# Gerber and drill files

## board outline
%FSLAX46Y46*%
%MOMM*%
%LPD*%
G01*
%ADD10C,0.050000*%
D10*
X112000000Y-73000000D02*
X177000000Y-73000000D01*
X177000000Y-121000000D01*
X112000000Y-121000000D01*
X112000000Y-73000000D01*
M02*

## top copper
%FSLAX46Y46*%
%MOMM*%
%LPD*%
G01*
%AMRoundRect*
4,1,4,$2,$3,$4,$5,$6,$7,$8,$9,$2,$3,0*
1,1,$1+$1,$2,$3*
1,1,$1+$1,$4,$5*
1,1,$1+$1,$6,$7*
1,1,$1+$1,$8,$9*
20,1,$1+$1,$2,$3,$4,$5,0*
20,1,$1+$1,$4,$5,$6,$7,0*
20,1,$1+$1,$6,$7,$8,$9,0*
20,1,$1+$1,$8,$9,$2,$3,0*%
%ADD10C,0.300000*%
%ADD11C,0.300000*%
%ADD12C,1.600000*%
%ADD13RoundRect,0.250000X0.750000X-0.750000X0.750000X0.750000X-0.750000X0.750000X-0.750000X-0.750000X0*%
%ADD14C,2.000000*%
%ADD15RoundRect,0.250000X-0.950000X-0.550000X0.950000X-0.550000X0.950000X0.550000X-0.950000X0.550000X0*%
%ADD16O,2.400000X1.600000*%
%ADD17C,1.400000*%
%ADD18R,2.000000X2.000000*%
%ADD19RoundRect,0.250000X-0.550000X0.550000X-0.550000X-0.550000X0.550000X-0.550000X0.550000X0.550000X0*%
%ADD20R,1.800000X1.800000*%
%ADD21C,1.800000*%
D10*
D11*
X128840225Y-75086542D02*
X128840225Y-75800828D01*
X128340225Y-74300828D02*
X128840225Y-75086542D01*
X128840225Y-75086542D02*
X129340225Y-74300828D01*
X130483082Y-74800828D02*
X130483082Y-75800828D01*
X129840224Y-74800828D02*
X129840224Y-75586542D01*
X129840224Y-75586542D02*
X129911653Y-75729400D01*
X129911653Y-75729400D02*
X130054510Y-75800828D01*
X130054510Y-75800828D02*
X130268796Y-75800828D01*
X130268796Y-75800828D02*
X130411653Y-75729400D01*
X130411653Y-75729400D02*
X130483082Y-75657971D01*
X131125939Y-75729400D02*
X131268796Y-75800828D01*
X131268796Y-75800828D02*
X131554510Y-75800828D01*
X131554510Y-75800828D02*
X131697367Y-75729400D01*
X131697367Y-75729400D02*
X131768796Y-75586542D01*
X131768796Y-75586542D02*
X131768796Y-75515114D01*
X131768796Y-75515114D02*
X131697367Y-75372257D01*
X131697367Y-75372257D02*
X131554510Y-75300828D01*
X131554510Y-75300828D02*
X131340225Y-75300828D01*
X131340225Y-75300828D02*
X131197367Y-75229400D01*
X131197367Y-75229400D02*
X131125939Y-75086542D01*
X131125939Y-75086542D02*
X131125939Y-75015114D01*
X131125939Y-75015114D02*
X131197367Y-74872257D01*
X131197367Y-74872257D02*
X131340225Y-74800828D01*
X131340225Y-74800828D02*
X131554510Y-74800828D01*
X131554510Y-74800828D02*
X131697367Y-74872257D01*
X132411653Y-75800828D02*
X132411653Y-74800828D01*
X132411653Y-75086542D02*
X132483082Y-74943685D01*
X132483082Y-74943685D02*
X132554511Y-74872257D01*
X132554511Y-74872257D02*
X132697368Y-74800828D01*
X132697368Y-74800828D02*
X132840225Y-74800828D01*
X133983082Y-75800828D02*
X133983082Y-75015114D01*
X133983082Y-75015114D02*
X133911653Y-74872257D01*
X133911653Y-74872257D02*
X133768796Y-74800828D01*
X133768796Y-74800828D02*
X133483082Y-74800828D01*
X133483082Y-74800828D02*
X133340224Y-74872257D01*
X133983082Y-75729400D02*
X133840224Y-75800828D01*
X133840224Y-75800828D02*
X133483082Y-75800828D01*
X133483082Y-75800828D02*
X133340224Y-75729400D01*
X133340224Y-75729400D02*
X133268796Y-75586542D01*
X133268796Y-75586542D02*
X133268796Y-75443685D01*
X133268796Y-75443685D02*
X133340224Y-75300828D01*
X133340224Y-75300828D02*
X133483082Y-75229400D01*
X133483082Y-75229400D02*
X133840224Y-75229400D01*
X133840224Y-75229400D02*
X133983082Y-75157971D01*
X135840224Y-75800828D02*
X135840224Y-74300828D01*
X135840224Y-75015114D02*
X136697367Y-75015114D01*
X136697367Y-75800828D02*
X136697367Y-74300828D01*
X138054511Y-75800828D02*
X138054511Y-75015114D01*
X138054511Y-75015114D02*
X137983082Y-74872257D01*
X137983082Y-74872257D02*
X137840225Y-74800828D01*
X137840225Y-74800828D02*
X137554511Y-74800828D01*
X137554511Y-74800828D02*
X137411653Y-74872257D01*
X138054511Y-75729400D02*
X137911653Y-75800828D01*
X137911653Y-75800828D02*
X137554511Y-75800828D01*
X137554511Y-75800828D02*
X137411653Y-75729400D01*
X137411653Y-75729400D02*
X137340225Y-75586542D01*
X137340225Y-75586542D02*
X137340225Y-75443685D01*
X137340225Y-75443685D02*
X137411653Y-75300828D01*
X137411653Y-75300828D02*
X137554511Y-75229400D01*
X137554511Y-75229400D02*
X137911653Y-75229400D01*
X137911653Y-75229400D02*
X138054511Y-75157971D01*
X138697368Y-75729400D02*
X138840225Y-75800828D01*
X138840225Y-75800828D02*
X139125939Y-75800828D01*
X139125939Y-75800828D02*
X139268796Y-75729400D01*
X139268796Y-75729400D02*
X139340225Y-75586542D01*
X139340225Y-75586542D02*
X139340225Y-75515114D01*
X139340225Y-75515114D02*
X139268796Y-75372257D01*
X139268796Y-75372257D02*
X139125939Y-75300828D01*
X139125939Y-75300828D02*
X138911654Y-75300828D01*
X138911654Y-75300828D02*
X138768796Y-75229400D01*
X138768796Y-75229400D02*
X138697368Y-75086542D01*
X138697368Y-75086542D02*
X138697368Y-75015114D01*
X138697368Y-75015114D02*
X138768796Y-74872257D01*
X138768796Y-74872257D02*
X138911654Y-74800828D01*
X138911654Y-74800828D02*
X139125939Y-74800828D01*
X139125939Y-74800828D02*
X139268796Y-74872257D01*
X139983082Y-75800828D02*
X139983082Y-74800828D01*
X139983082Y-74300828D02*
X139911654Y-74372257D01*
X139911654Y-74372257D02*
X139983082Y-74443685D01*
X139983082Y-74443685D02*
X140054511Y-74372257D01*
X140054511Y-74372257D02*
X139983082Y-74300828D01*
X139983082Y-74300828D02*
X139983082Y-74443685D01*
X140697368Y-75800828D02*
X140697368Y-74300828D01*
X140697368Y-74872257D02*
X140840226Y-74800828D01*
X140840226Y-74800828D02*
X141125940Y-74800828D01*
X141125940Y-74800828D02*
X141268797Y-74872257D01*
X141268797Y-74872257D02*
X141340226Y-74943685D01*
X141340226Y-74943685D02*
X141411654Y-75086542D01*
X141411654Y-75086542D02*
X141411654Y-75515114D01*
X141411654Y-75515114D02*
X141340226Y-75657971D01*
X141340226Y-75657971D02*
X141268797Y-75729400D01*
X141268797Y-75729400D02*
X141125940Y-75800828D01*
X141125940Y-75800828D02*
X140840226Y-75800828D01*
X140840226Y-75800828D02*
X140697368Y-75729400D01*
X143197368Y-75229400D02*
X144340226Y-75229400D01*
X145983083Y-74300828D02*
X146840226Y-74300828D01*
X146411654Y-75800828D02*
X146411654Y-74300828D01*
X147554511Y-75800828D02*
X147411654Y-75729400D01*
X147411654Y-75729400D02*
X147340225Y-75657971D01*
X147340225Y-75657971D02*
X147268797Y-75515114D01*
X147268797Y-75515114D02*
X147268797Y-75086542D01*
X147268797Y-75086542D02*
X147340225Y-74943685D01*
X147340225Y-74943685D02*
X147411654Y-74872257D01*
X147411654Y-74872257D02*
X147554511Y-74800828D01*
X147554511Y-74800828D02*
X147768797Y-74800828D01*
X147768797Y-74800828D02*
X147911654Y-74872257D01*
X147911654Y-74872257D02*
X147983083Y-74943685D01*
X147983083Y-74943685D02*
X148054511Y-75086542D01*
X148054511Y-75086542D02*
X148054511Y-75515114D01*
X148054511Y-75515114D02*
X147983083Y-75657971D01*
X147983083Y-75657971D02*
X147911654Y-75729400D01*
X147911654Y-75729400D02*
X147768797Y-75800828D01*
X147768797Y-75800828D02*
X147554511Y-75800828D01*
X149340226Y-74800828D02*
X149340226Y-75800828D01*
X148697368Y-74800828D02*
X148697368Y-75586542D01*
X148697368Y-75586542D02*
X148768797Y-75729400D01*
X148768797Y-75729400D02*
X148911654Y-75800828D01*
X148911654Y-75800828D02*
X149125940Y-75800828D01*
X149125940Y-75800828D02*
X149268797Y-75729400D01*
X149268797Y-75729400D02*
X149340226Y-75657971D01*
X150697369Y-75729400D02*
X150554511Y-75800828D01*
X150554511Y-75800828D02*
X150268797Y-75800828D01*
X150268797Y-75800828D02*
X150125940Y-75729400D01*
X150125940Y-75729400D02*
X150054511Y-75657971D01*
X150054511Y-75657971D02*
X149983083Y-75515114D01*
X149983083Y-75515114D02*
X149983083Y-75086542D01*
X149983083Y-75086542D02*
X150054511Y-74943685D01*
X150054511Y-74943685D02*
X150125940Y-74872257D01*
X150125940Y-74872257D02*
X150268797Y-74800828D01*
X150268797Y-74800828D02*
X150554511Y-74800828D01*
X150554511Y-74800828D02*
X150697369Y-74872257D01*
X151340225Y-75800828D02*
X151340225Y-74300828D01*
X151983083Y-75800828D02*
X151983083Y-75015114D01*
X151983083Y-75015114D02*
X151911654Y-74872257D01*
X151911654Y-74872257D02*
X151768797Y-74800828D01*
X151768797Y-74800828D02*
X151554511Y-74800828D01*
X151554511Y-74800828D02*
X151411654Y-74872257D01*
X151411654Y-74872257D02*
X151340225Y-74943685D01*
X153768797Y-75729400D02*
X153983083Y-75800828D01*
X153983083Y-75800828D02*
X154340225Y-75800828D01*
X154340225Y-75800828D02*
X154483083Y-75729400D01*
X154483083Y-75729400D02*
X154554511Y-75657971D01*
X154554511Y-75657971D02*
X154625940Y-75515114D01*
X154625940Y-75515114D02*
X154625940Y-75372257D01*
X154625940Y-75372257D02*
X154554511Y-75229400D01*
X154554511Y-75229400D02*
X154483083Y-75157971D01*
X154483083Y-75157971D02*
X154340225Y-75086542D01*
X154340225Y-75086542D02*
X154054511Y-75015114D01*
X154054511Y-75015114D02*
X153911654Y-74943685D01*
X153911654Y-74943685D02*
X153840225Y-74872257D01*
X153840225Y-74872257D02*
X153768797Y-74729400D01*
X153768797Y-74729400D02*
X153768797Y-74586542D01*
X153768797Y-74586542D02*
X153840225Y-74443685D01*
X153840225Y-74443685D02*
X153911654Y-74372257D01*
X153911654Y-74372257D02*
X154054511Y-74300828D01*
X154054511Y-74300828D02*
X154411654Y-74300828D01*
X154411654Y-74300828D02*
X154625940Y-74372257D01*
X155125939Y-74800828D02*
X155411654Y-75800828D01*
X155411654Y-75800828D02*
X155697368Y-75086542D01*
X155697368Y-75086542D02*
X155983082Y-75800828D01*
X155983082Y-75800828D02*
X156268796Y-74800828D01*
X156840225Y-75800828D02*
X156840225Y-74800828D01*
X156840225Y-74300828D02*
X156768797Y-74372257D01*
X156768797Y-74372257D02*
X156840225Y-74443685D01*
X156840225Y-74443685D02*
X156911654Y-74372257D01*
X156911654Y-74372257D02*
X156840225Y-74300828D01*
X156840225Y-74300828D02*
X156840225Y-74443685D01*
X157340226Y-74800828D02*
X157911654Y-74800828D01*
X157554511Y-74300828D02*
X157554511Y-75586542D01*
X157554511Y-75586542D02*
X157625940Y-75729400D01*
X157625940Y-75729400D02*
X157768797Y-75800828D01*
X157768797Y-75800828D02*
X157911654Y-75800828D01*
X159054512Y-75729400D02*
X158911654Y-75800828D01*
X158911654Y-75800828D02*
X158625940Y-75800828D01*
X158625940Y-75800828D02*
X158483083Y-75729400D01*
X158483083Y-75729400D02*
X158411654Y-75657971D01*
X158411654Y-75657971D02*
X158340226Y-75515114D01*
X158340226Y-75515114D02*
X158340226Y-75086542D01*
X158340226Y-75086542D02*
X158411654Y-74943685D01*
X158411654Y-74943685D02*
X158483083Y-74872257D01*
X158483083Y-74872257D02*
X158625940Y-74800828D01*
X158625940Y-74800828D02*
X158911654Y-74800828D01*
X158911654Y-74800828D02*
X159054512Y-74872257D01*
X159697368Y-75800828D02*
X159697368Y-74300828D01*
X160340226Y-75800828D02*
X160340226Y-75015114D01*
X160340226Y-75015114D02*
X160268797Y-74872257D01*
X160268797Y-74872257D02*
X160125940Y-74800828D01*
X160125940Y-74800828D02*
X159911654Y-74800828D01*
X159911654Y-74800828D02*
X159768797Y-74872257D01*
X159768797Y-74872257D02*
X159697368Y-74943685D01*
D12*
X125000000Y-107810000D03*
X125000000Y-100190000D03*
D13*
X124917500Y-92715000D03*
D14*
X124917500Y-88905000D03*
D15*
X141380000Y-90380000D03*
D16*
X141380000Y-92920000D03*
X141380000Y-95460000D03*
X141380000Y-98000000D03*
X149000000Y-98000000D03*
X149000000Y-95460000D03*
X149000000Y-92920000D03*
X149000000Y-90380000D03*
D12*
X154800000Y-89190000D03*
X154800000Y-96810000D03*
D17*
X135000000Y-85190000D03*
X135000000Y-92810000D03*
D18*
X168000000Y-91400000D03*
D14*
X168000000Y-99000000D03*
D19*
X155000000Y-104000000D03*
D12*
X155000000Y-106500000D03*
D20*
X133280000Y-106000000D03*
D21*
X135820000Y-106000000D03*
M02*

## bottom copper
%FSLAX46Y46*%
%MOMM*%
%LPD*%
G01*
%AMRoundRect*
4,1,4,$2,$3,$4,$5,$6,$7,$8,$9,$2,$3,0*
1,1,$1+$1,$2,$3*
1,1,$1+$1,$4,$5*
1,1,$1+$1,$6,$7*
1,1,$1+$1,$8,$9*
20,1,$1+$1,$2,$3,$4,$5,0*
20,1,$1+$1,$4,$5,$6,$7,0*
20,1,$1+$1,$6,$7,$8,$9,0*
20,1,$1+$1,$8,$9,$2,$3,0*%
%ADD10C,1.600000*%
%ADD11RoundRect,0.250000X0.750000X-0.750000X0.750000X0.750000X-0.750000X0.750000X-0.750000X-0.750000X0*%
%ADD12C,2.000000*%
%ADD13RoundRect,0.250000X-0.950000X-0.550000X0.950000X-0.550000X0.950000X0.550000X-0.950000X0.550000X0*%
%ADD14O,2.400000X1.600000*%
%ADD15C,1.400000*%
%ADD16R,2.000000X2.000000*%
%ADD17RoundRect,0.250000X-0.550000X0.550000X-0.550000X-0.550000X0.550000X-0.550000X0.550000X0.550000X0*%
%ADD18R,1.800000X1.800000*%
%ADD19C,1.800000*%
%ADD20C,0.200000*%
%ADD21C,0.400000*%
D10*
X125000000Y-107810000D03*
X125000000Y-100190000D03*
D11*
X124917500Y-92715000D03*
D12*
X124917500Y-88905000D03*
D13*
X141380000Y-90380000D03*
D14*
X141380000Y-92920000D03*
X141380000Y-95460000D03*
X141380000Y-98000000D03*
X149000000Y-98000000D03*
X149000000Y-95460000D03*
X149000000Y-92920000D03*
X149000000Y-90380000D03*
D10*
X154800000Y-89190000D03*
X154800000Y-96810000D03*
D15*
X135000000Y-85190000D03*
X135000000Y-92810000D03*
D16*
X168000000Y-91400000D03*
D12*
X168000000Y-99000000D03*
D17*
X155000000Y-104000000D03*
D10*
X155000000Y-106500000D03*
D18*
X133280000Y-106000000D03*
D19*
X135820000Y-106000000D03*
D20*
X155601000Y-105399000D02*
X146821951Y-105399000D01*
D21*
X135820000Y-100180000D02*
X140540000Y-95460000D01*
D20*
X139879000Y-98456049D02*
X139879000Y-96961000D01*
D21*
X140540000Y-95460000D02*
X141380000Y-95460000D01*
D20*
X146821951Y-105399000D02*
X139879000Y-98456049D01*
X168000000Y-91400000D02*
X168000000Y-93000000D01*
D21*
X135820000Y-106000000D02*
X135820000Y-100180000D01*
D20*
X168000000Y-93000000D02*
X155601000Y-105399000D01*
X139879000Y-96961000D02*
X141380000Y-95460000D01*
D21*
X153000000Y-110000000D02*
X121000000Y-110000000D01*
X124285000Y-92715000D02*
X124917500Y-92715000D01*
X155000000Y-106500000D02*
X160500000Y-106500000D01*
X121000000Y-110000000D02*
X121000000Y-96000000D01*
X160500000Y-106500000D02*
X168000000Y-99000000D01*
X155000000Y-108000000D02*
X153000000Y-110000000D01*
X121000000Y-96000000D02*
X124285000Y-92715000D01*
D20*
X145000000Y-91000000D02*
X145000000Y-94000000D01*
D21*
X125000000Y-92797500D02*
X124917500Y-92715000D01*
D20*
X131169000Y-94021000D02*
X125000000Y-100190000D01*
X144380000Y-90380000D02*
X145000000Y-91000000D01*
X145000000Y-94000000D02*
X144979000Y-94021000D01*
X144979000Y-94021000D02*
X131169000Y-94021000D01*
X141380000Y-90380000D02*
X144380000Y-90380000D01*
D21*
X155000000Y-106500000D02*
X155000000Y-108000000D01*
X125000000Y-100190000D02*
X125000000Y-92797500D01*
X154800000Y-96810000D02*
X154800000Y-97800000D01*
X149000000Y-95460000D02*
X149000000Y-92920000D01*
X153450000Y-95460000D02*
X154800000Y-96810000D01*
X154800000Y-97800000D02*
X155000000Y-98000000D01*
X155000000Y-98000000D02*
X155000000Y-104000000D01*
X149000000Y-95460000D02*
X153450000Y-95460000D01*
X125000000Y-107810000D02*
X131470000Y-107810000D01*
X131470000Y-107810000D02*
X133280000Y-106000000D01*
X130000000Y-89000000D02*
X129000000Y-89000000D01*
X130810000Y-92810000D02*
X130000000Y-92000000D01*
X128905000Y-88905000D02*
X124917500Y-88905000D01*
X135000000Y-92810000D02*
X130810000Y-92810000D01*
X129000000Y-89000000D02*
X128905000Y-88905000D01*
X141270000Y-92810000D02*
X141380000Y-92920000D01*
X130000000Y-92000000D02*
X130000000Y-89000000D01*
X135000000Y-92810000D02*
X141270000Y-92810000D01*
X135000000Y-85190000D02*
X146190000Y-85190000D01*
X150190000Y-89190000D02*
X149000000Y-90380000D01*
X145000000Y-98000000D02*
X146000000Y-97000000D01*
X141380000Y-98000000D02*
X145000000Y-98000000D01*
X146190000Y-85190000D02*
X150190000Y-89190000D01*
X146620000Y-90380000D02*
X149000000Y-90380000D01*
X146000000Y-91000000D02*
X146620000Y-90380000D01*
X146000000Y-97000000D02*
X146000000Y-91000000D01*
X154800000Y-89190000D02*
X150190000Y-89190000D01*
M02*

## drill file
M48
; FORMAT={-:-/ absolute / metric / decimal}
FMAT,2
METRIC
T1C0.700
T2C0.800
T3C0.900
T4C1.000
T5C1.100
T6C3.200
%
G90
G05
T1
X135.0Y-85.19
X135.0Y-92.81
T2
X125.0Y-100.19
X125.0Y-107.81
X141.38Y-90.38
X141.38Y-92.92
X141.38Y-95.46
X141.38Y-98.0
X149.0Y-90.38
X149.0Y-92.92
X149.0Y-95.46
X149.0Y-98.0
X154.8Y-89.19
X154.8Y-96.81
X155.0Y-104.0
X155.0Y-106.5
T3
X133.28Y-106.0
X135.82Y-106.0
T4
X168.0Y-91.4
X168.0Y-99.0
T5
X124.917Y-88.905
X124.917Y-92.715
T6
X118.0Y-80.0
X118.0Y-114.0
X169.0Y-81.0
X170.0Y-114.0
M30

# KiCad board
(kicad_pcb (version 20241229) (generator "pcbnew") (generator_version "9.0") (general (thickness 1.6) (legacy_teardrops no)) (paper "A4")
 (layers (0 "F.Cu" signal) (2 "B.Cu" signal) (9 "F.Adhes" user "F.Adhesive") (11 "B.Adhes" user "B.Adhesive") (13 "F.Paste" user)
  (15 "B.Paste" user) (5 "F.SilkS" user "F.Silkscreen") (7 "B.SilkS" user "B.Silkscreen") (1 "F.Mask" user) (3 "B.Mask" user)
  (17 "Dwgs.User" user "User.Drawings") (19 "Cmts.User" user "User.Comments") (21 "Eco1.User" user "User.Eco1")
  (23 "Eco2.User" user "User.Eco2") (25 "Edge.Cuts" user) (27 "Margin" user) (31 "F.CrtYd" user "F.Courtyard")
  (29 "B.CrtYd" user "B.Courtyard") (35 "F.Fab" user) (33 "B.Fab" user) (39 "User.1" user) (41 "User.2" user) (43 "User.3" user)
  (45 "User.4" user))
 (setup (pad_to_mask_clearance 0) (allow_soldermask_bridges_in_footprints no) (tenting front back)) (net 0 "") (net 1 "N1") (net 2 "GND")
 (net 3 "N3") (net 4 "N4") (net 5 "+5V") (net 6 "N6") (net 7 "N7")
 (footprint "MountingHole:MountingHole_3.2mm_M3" (layer "F.Cu") (at 169 81)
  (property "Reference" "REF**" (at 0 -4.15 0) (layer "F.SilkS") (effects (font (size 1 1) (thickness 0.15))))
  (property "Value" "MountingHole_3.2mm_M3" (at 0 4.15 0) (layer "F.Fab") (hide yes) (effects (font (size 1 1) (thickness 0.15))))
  (pad "" np_thru_hole circle (at 0 0) (size 3.2 3.2) (drill 3.2) (layers "*.Cu" "*.Mask")))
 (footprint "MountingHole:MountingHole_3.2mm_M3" (layer "F.Cu") (at 118 114)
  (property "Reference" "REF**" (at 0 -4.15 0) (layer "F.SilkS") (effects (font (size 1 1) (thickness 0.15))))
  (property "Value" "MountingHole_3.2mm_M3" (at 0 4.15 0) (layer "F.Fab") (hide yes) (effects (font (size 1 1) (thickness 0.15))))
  (pad "" np_thru_hole circle (at 0 0) (size 3.2 3.2) (drill 3.2) (layers "*.Cu" "*.Mask")))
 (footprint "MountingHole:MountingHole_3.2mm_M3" (layer "F.Cu") (at 118 80)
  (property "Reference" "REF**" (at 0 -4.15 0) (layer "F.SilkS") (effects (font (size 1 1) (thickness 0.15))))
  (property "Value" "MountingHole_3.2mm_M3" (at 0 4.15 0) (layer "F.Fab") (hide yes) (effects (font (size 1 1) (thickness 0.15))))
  (pad "" np_thru_hole circle (at 0 0) (size 3.2 3.2) (drill 3.2) (layers "*.Cu" "*.Mask")))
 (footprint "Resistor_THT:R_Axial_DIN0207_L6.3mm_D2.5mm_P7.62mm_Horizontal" (layer "F.Cu") (at 125 107.81 90)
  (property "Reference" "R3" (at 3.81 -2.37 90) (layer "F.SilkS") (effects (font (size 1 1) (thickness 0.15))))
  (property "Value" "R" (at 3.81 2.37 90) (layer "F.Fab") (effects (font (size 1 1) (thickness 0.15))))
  (pad "1" thru_hole circle (at 0 0 90) (size 1.6 1.6) (drill 0.8) (layers "*.Cu" "*.Mask") (remove_unused_layers no) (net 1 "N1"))
  (pad "2" thru_hole circle (at 7.62 0 90) (size 1.6 1.6) (drill 0.8) (layers "*.Cu" "*.Mask") (remove_unused_layers no) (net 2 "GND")))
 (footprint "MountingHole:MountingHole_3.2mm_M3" (layer "F.Cu") (at 170 114)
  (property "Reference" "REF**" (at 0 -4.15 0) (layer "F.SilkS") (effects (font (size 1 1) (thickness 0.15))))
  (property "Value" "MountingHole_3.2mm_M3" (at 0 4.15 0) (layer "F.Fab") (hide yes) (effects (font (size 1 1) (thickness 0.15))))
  (pad "" np_thru_hole circle (at 0 0) (size 3.2 3.2) (drill 3.2) (layers "*.Cu" "*.Mask")))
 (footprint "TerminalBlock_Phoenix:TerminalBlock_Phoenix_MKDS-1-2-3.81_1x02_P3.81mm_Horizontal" (layer "F.Cu") (at 124.9175 92.715 90)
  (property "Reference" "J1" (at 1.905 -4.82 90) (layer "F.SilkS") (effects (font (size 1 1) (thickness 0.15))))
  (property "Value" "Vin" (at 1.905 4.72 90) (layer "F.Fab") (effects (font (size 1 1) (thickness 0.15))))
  (pad "1" thru_hole roundrect (at 0 0 90) (size 2 2) (drill 1.1) (layers "*.Cu" "*.Mask") (remove_unused_layers no)
   (roundrect_rratio 0.125) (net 2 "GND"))
  (pad "2" thru_hole circle (at 3.81 0 90) (size 2 2) (drill 1.1) (layers "*.Cu" "*.Mask") (remove_unused_layers no) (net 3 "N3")))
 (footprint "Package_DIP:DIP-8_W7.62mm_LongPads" (layer "F.Cu") (at 141.38 90.38)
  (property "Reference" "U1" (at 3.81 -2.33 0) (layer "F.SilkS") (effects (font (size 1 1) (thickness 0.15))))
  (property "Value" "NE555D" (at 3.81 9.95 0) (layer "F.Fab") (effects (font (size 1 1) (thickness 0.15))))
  (pad "1" thru_hole roundrect (at 0 0) (size 2.4 1.6) (drill 0.8) (layers "*.Cu" "*.Mask") (remove_unused_layers no)
   (roundrect_rratio 0.15625) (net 2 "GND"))
  (pad "2" thru_hole oval (at 0 2.54) (size 2.4 1.6) (drill 0.8) (layers "*.Cu" "*.Mask") (remove_unused_layers no) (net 3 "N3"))
  (pad "3" thru_hole oval (at 0 5.08) (size 2.4 1.6) (drill 0.8) (layers "*.Cu" "*.Mask") (remove_unused_layers no) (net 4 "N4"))
  (pad "4" thru_hole oval (at 0 7.62) (size 2.4 1.6) (drill 0.8) (layers "*.Cu" "*.Mask") (remove_unused_layers no) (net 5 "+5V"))
  (pad "5" thru_hole oval (at 7.62 7.62) (size 2.4 1.6) (drill 0.8) (layers "*.Cu" "*.Mask") (remove_unused_layers no) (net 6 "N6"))
  (pad "6" thru_hole oval (at 7.62 5.08) (size 2.4 1.6) (drill 0.8) (layers "*.Cu" "*.Mask") (remove_unused_layers no) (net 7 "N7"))
  (pad "7" thru_hole oval (at 7.62 2.54) (size 2.4 1.6) (drill 0.8) (layers "*.Cu" "*.Mask") (remove_unused_layers no) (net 7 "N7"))
  (pad "8" thru_hole oval (at 7.62 0) (size 2.4 1.6) (drill 0.8) (layers "*.Cu" "*.Mask") (remove_unused_layers no) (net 5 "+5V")))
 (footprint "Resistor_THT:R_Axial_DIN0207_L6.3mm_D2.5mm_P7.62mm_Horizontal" (layer "F.Cu") (at 154.8 89.19 -90)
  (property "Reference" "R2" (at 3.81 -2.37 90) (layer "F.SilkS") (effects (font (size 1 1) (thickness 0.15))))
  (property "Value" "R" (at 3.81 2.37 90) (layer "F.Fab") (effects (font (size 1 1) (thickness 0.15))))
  (pad "1" thru_hole circle (at 0 0 270) (size 1.6 1.6) (drill 0.8) (layers "*.Cu" "*.Mask") (remove_unused_layers no) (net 5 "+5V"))
  (pad "2" thru_hole circle (at 7.62 0 270) (size 1.6 1.6) (drill 0.8) (layers "*.Cu" "*.Mask") (remove_unused_layers no) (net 7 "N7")))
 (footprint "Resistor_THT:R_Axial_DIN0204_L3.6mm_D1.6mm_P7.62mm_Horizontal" (layer "F.Cu") (at 135 85.19 -90)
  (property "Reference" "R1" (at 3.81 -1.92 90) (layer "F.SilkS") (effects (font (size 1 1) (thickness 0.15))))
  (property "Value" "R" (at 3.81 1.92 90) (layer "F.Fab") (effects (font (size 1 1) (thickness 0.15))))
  (pad "1" thru_hole circle (at 0 0 270) (size 1.4 1.4) (drill 0.7) (layers "*.Cu" "*.Mask") (remove_unused_layers no) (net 5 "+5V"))
  (pad "2" thru_hole circle (at 7.62 0 270) (size 1.4 1.4) (drill 0.7) (layers "*.Cu" "*.Mask") (remove_unused_layers no) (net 3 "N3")))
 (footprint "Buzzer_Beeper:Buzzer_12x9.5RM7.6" (layer "F.Cu") (at 168 91.4 -90)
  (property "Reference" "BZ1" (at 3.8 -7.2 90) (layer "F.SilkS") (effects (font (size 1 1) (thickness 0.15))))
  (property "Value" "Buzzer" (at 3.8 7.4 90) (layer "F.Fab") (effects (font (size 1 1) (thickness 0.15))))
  (pad "1" thru_hole rect (at 0 0 270) (size 2 2) (drill 1) (layers "*.Cu" "*.Mask") (remove_unused_layers no) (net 4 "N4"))
  (pad "2" thru_hole circle (at 7.6 0 270) (size 2 2) (drill 1) (layers "*.Cu" "*.Mask") (remove_unused_layers no) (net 2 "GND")))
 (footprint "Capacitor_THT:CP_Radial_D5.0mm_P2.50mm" (layer "F.Cu") (at 155 104 -90)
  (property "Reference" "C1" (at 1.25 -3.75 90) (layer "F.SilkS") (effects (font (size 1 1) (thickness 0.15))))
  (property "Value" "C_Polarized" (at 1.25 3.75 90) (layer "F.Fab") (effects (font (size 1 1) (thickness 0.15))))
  (pad "1" thru_hole roundrect (at 0 0 270) (size 1.6 1.6) (drill 0.8) (layers "*.Cu" "*.Mask") (remove_unused_layers no)
   (roundrect_rratio 0.15625) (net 7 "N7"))
  (pad "2" thru_hole circle (at 2.5 0 270) (size 1.6 1.6) (drill 0.8) (layers "*.Cu" "*.Mask") (remove_unused_layers no) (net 2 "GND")))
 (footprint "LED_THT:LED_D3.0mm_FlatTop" (layer "F.Cu") (at 133.28 106)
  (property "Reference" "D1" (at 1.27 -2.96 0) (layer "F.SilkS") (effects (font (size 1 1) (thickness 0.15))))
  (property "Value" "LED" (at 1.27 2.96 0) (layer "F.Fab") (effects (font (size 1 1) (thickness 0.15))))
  (pad "1" thru_hole rect (at 0 0) (size 1.8 1.8) (drill 0.9) (layers "*.Cu" "*.Mask") (remove_unused_layers no) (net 1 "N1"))
  (pad "2" thru_hole circle (at 2.54 0) (size 1.8 1.8) (drill 0.9) (layers "*.Cu" "*.Mask") (remove_unused_layers no) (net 4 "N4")))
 (gr_poly (pts (xy 112 73) (xy 177 73) (xy 177 121) (xy 112 121)) (stroke (width 0.05) (type solid)) (fill no) (layer "Edge.Cuts"))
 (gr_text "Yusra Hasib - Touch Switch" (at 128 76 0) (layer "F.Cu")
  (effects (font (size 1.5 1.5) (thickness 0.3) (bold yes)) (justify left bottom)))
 (segment (start 155.601 105.399) (end 146.821951 105.399) (width 0.2) (layer "B.Cu") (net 4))
 (segment (start 135.82 100.18) (end 140.54 95.46) (width 0.4) (layer "B.Cu") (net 4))
 (segment (start 139.879 98.456049) (end 139.879 96.961) (width 0.2) (layer "B.Cu") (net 4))
 (segment (start 140.54 95.46) (end 141.38 95.46) (width 0.4) (layer "B.Cu") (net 4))
 (segment (start 146.821951 105.399) (end 139.879 98.456049) (width 0.2) (layer "B.Cu") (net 4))
 (segment (start 168 91.4) (end 168 93) (width 0.2) (layer "B.Cu") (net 4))
 (segment (start 135.82 106) (end 135.82 100.18) (width 0.4) (layer "B.Cu") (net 4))
 (segment (start 168 93) (end 155.601 105.399) (width 0.2) (layer "B.Cu") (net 4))
 (segment (start 139.879 96.961) (end 141.38 95.46) (width 0.2) (layer "B.Cu") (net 4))
 (segment (start 153 110) (end 121 110) (width 0.4) (layer "B.Cu") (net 2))
 (segment (start 124.285 92.715) (end 124.9175 92.715) (width 0.4) (layer "B.Cu") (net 2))
 (segment (start 155 106.5) (end 160.5 106.5) (width 0.4) (layer "B.Cu") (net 2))
 (segment (start 121 110) (end 121 96) (width 0.4) (layer "B.Cu") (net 2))
 (segment (start 160.5 106.5) (end 168 99) (width 0.4) (layer "B.Cu") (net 2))
 (segment (start 155 108) (end 153 110) (width 0.4) (layer "B.Cu") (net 2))
 (segment (start 121 96) (end 124.285 92.715) (width 0.4) (layer "B.Cu") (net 2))
 (segment (start 145 91) (end 145 94) (width 0.2) (layer "B.Cu") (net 2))
 (segment (start 125 92.7975) (end 124.9175 92.715) (width 0.4) (layer "B.Cu") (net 2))
 (segment (start 131.169 94.021) (end 125 100.19) (width 0.2) (layer "B.Cu") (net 2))
 (segment (start 144.38 90.38) (end 145 91) (width 0.2) (layer "B.Cu") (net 2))
 (segment (start 145 94) (end 144.979 94.021) (width 0.2) (layer "B.Cu") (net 2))
 (segment (start 144.979 94.021) (end 131.169 94.021) (width 0.2) (layer "B.Cu") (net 2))
 (segment (start 141.38 90.38) (end 144.38 90.38) (width 0.2) (layer "B.Cu") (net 2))
 (segment (start 155 106.5) (end 155 108) (width 0.4) (layer "B.Cu") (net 2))
 (segment (start 125 100.19) (end 125 92.7975) (width 0.4) (layer "B.Cu") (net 2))
 (segment (start 154.8 96.81) (end 154.8 97.8) (width 0.4) (layer "B.Cu") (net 7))
 (segment (start 149 95.46) (end 149 92.92) (width 0.4) (layer "B.Cu") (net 7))
 (segment (start 153.45 95.46) (end 154.8 96.81) (width 0.4) (layer "B.Cu") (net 7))
 (segment (start 154.8 97.8) (end 155 98) (width 0.4) (layer "B.Cu") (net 7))
 (segment (start 155 98) (end 155 104) (width 0.4) (layer "B.Cu") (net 7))
 (segment (start 149 95.46) (end 153.45 95.46) (width 0.4) (layer "B.Cu") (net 7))
 (segment (start 125 107.81) (end 131.47 107.81) (width 0.4) (layer "B.Cu") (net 1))
 (segment (start 131.47 107.81) (end 133.28 106) (width 0.4) (layer "B.Cu") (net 1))
 (segment (start 130 89) (end 129 89) (width 0.4) (layer "B.Cu") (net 3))
 (segment (start 130.81 92.81) (end 130 92) (width 0.4) (layer "B.Cu") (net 3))
 (segment (start 128.905 88.905) (end 124.9175 88.905) (width 0.4) (layer "B.Cu") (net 3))
 (segment (start 135 92.81) (end 130.81 92.81) (width 0.4) (layer "B.Cu") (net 3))
 (segment (start 129 89) (end 128.905 88.905) (width 0.4) (layer "B.Cu") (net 3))
 (segment (start 141.27 92.81) (end 141.38 92.92) (width 0.4) (layer "B.Cu") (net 3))
 (segment (start 130 92) (end 130 89) (width 0.4) (layer "B.Cu") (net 3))
 (segment (start 135 92.81) (end 141.27 92.81) (width 0.4) (layer "B.Cu") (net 3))
 (segment (start 135 85.19) (end 146.19 85.19) (width 0.4) (layer "B.Cu") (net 5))
 (segment (start 150.19 89.19) (end 149 90.38) (width 0.4) (layer "B.Cu") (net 5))
 (segment (start 145 98) (end 146 97) (width 0.4) (layer "B.Cu") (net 5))
 (segment (start 141.38 98) (end 145 98) (width 0.4) (layer "B.Cu") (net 5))
 (segment (start 146.19 85.19) (end 150.19 89.19) (width 0.4) (layer "B.Cu") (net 5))
 (segment (start 146.62 90.38) (end 149 90.38) (width 0.4) (layer "B.Cu") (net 5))
 (segment (start 146 91) (end 146.62 90.38) (width 0.4) (layer "B.Cu") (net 5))
 (segment (start 146 97) (end 146 91) (width 0.4) (layer "B.Cu") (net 5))
 (segment (start 154.8 89.19) (end 150.19 89.19) (width 0.4) (layer "B.Cu") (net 5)))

